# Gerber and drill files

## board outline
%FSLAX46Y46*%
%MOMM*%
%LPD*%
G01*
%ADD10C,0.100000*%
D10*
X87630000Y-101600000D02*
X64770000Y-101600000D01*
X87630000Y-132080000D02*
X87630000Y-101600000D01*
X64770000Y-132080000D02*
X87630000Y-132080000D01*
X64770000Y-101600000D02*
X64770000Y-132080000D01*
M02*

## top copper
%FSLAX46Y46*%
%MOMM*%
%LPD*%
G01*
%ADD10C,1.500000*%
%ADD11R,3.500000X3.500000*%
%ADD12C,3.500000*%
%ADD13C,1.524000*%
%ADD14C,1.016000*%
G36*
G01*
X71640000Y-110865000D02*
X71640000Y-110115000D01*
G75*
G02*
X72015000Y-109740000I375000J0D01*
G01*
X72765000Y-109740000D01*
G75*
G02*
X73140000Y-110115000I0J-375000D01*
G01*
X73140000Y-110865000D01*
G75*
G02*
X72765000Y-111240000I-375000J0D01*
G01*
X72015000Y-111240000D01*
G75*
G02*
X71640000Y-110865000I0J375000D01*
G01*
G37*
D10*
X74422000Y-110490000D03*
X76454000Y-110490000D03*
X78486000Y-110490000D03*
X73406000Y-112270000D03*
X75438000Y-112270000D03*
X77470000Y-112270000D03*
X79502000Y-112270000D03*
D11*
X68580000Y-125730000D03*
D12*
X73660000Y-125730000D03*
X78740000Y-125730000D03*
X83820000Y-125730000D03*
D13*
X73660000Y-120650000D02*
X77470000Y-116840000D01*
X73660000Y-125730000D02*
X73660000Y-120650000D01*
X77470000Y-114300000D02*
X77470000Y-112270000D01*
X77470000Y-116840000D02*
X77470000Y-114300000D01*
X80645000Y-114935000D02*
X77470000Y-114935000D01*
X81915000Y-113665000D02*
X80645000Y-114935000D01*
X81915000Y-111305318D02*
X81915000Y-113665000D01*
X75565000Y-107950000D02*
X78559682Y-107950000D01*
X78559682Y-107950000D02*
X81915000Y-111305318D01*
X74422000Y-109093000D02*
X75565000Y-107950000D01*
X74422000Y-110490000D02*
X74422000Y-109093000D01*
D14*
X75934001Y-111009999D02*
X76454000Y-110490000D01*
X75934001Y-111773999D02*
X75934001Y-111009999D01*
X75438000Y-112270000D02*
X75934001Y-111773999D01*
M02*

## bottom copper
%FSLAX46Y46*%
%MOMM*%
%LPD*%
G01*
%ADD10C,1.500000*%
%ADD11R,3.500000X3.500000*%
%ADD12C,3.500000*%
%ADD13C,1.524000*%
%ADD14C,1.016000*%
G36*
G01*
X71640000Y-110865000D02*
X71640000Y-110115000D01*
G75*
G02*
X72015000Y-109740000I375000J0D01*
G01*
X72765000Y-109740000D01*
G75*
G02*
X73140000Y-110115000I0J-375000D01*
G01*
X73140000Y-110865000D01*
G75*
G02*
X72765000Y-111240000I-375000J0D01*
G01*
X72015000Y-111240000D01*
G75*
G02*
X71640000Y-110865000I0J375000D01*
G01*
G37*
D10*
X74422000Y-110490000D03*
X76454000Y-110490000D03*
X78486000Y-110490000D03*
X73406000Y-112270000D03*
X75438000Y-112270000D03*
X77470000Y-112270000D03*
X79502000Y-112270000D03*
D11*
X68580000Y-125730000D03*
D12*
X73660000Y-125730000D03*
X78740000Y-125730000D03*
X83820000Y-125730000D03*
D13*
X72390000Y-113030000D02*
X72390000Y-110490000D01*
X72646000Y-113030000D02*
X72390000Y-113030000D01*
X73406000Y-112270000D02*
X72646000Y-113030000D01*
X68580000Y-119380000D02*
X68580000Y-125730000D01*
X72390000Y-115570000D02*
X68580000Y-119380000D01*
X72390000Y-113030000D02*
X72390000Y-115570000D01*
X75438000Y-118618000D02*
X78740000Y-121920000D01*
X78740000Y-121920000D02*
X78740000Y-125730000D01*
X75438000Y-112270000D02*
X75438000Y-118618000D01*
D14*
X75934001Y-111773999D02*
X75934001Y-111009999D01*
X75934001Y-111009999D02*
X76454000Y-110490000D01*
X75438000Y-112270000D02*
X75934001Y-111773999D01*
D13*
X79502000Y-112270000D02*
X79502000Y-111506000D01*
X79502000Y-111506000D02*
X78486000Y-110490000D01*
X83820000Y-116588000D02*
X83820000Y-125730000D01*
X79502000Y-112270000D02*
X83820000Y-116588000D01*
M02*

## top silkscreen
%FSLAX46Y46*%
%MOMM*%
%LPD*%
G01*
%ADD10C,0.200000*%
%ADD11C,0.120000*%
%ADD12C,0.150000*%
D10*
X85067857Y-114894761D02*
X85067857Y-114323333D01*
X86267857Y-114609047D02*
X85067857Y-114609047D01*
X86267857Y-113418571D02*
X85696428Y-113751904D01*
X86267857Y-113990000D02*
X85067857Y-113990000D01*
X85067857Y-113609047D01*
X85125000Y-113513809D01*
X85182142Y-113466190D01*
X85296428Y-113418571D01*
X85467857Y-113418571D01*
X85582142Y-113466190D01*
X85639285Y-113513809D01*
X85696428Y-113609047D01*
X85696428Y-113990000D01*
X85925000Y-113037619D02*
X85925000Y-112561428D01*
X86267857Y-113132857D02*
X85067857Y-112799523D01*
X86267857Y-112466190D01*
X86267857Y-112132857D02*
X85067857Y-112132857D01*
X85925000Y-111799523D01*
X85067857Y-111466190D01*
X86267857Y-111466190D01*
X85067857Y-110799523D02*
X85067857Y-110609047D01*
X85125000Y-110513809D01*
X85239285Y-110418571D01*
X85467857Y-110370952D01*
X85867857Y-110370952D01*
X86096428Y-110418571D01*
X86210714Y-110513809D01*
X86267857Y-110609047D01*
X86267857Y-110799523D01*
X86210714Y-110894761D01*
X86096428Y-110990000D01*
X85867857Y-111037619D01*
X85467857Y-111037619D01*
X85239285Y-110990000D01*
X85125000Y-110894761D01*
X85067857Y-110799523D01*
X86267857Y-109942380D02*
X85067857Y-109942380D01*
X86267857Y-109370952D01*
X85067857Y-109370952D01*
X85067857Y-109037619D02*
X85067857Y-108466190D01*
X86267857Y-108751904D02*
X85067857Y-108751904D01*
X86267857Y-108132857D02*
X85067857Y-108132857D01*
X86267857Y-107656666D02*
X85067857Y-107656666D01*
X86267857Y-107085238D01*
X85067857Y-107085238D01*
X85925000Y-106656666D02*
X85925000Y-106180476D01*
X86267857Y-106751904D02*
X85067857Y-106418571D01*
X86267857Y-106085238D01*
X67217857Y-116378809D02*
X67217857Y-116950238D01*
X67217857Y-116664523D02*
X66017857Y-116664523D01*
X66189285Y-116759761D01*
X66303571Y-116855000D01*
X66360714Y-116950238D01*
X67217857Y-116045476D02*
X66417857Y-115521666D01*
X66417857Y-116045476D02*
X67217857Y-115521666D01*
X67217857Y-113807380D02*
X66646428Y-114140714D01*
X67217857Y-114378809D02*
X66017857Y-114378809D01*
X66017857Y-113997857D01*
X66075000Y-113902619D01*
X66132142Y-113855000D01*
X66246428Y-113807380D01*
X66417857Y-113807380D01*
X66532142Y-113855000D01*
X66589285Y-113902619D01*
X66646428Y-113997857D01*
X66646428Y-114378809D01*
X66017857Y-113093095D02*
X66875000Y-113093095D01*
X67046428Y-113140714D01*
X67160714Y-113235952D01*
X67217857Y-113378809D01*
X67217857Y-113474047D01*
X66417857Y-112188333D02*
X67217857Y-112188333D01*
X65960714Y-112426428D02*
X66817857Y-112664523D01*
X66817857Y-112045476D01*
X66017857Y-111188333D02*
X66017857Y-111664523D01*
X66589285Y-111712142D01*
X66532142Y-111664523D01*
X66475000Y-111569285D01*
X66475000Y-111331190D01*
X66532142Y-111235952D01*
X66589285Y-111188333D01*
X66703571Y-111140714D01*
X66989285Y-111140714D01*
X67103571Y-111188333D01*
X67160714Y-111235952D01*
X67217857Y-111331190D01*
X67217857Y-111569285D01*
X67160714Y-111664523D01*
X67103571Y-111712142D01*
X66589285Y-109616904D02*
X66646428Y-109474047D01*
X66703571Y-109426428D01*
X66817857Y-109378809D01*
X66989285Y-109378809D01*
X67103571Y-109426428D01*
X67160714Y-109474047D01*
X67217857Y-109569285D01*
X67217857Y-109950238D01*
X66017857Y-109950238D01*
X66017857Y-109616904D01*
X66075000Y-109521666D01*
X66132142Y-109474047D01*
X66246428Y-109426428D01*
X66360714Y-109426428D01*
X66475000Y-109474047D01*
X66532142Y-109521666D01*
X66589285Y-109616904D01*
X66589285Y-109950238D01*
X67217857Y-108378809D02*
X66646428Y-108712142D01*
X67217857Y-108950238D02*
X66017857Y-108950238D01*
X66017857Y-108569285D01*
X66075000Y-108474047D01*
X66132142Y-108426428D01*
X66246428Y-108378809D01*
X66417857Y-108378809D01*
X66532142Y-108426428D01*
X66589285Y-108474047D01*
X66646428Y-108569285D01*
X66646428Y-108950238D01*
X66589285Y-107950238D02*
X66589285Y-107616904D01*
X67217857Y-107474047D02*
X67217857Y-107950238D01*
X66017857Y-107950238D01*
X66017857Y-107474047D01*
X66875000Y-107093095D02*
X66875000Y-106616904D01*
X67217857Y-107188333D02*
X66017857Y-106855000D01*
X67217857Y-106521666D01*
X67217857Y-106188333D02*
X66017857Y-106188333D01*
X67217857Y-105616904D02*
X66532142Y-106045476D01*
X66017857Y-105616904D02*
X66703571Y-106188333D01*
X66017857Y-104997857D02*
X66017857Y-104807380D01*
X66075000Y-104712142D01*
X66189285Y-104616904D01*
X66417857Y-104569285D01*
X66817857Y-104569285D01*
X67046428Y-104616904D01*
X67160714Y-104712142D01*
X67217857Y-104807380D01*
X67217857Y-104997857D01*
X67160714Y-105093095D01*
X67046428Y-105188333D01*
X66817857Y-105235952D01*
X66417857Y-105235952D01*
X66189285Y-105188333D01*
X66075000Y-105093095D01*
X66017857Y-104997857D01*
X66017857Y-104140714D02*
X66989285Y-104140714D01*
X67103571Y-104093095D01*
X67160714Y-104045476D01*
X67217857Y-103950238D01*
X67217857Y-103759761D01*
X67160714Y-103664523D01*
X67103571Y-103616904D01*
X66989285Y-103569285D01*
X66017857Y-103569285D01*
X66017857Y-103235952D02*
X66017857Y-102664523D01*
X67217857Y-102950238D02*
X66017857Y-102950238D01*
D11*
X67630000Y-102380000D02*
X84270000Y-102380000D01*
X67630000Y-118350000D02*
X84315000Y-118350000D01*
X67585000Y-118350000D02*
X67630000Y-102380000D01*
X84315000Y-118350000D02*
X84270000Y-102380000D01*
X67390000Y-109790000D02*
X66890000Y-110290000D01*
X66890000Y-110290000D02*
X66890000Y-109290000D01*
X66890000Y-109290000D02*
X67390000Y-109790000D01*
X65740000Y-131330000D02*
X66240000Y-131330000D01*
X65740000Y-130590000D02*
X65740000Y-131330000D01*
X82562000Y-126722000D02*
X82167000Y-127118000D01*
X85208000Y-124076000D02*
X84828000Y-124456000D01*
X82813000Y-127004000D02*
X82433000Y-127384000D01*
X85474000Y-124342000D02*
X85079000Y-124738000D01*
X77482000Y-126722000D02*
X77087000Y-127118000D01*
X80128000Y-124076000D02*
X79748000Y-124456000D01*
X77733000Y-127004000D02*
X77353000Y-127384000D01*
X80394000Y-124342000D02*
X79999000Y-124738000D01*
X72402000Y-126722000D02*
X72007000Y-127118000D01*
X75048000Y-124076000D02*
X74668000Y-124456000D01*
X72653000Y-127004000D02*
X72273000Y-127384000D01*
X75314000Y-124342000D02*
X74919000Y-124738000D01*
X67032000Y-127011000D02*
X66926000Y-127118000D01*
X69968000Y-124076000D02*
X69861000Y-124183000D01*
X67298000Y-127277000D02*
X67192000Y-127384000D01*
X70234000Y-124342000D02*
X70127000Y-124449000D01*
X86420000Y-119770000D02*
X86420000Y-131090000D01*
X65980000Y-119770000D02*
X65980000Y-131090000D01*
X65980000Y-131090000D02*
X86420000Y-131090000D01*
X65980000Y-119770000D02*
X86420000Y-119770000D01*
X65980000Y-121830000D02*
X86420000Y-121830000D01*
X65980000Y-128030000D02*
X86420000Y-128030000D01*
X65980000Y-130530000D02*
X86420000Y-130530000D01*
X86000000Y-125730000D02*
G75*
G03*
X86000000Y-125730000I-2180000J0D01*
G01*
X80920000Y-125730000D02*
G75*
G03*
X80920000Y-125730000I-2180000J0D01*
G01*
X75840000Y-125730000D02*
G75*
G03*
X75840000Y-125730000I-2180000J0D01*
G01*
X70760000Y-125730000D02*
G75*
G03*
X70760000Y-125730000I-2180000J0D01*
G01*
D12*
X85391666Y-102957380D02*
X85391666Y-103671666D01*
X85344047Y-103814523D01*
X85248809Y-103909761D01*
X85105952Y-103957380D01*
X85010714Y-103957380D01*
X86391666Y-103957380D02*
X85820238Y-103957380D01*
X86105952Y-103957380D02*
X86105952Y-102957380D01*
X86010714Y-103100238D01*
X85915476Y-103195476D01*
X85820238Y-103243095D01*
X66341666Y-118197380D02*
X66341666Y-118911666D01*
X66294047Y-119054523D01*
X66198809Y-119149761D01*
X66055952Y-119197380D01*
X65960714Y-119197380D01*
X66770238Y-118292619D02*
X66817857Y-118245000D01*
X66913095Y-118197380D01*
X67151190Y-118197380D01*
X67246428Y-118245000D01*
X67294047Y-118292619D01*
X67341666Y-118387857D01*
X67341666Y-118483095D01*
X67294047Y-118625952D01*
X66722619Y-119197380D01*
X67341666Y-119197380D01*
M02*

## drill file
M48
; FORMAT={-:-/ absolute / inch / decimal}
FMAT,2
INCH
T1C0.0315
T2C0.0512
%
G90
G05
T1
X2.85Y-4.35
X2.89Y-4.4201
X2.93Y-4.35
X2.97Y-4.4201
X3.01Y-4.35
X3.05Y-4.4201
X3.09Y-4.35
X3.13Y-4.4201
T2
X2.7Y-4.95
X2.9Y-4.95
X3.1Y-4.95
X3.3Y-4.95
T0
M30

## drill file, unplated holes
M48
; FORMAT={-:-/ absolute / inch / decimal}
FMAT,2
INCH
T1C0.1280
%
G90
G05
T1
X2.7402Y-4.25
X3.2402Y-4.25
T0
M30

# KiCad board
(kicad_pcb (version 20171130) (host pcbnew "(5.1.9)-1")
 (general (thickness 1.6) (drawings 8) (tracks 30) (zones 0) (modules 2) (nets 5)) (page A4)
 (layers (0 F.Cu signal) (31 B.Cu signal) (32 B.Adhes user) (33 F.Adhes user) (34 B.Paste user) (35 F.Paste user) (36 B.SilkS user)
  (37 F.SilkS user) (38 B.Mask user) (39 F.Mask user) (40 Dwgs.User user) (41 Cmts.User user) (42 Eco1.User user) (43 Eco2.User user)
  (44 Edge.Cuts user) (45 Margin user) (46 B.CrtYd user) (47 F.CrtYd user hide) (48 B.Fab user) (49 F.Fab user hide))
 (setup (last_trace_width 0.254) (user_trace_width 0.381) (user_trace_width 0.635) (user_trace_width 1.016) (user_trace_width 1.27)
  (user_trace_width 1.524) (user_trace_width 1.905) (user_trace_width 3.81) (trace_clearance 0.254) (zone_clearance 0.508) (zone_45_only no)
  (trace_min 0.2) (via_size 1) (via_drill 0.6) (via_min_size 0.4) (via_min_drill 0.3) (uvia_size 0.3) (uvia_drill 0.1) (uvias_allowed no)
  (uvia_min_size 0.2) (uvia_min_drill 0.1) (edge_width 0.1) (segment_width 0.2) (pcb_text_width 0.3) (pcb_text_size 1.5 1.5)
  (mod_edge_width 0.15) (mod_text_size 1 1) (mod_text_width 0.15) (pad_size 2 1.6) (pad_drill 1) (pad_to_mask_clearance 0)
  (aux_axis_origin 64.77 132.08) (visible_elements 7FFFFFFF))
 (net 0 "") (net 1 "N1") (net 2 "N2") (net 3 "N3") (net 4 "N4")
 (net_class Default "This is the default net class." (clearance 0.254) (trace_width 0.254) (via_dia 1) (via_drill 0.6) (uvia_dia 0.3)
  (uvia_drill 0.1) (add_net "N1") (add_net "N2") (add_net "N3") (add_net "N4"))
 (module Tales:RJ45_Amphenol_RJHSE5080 (layer F.Cu) (at 72.39 110.49)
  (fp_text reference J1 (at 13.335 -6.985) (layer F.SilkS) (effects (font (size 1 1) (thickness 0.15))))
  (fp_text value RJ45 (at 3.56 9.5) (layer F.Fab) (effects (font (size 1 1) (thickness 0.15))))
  (fp_line (start -4.76 -8.11) (end 11.88 -8.11) (layer F.SilkS) (width 0.12))
  (fp_line (start -4.76 7.86) (end 11.925 7.86) (layer F.SilkS) (width 0.12))
  (fp_line (start -4.805 7.86) (end -4.76 -8.11) (layer F.SilkS) (width 0.12))
  (fp_line (start 11.925 7.86) (end 11.88 -8.11) (layer F.SilkS) (width 0.12))
  (fp_line (start -5 -0.7) (end -5.5 -0.2) (layer F.SilkS) (width 0.12))
  (fp_line (start -5.5 -0.2) (end -5.5 -1.2) (layer F.SilkS) (width 0.12))
  (fp_line (start -5.5 -1.2) (end -5 -0.7) (layer F.SilkS) (width 0.12))
  (pad 1 thru_hole roundrect (at 0 0) (size 1.5 1.5) (drill 0.8) (layers *.Cu *.Mask) (roundrect_rratio 0.25) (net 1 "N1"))
  (pad 3 thru_hole circle (at 2.032 0) (size 1.5 1.5) (drill 0.8) (layers *.Cu *.Mask) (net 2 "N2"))
  (pad 5 thru_hole circle (at 4.064 0) (size 1.5 1.5) (drill 0.8) (layers *.Cu *.Mask) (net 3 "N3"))
  (pad 7 thru_hole circle (at 6.096 0) (size 1.5 1.5) (drill 0.8) (layers *.Cu *.Mask) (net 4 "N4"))
  (pad 2 thru_hole circle (at 1.016 1.78) (size 1.5 1.5) (drill 0.8) (layers *.Cu *.Mask) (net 1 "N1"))
  (pad 4 thru_hole circle (at 3.048 1.78) (size 1.5 1.5) (drill 0.8) (layers *.Cu *.Mask) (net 3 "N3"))
  (pad 6 thru_hole circle (at 5.08 1.78) (size 1.5 1.5) (drill 0.8) (layers *.Cu *.Mask) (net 2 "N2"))
  (pad 8 thru_hole circle (at 7.112 1.78) (size 1.5 1.5) (drill 0.8) (layers *.Cu *.Mask) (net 4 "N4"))
  (pad "" np_thru_hole circle (at -2.79 -2.54) (size 3.25 3.25) (drill 3.25) (layers *.Cu *.Mask))
  (pad "" np_thru_hole circle (at 9.91 -2.54) (size 3.25 3.25) (drill 3.25) (layers *.Cu *.Mask)))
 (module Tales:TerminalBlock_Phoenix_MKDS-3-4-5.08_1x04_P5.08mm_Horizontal (layer F.Cu) (at 68.58 125.73)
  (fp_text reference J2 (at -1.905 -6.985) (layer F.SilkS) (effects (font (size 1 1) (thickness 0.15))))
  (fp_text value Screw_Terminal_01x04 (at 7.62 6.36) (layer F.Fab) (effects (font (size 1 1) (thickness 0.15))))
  (fp_line (start -2.84 5.6) (end -2.34 5.6) (layer F.SilkS) (width 0.12))
  (fp_line (start -2.84 4.86) (end -2.84 5.6) (layer F.SilkS) (width 0.12))
  (fp_line (start 13.982 0.992) (end 13.587 1.388) (layer F.SilkS) (width 0.12))
  (fp_line (start 16.628 -1.654) (end 16.248 -1.274) (layer F.SilkS) (width 0.12))
  (fp_line (start 14.233 1.274) (end 13.853 1.654) (layer F.SilkS) (width 0.12))
  (fp_line (start 16.894 -1.388) (end 16.499 -0.992) (layer F.SilkS) (width 0.12))
  (fp_line (start 8.902 0.992) (end 8.507 1.388) (layer F.SilkS) (width 0.12))
  (fp_line (start 11.548 -1.654) (end 11.168 -1.274) (layer F.SilkS) (width 0.12))
  (fp_line (start 9.153 1.274) (end 8.773 1.654) (layer F.SilkS) (width 0.12))
  (fp_line (start 11.814 -1.388) (end 11.419 -0.992) (layer F.SilkS) (width 0.12))
  (fp_line (start 3.822 0.992) (end 3.427 1.388) (layer F.SilkS) (width 0.12))
  (fp_line (start 6.468 -1.654) (end 6.088 -1.274) (layer F.SilkS) (width 0.12))
  (fp_line (start 4.073 1.274) (end 3.693 1.654) (layer F.SilkS) (width 0.12))
  (fp_line (start 6.734 -1.388) (end 6.339 -0.992) (layer F.SilkS) (width 0.12))
  (fp_line (start -1.548 1.281) (end -1.654 1.388) (layer F.SilkS) (width 0.12))
  (fp_line (start 1.388 -1.654) (end 1.281 -1.547) (layer F.SilkS) (width 0.12))
  (fp_line (start -1.282 1.547) (end -1.388 1.654) (layer F.SilkS) (width 0.12))
  (fp_line (start 1.654 -1.388) (end 1.547 -1.281) (layer F.SilkS) (width 0.12))
  (fp_line (start 17.84 -5.96) (end 17.84 5.36) (layer F.SilkS) (width 0.12))
  (fp_line (start -2.6 -5.96) (end -2.6 5.36) (layer F.SilkS) (width 0.12))
  (fp_line (start -2.6 5.36) (end 17.84 5.36) (layer F.SilkS) (width 0.12))
  (fp_line (start -2.6 -5.96) (end 17.84 -5.96) (layer F.SilkS) (width 0.12))
  (fp_line (start -2.6 -3.9) (end 17.84 -3.9) (layer F.SilkS) (width 0.12))
  (fp_line (start -2.6 2.3) (end 17.84 2.3) (layer F.SilkS) (width 0.12))
  (fp_line (start -2.6 4.8) (end 17.84 4.8) (layer F.SilkS) (width 0.12))
  (fp_circle (center 15.24 0) (end 17.42 0) (layer F.SilkS) (width 0.12))
  (fp_circle (center 10.16 0) (end 12.34 0) (layer F.SilkS) (width 0.12))
  (fp_circle (center 5.08 0) (end 7.26 0) (layer F.SilkS) (width 0.12))
  (fp_circle (center 0 0) (end 2.18 0) (layer F.SilkS) (width 0.12))
  (pad 1 thru_hole rect (at 0 0) (size 3.5 3.5) (drill 1.3) (layers *.Cu *.Mask) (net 1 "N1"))
  (pad 2 thru_hole circle (at 5.08 0) (size 3.5 3.5) (drill 1.3) (layers *.Cu *.Mask) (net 2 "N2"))
  (pad 3 thru_hole circle (at 10.16 0) (size 3.5 3.5) (drill 1.3) (layers *.Cu *.Mask) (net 3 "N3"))
  (pad 4 thru_hole circle (at 15.24 0) (size 3.5 3.5) (drill 1.3) (layers *.Cu *.Mask) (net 4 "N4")))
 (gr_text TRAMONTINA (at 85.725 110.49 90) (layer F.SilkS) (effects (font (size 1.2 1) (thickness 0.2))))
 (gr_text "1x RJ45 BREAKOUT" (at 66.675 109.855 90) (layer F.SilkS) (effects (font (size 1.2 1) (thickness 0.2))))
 (gr_line (start 87.63 101.6) (end 64.77 101.6) (layer Edge.Cuts) (width 0.1))
 (gr_line (start 87.63 132.08) (end 87.63 101.6) (layer Edge.Cuts) (width 0.1))
 (gr_line (start 64.77 132.08) (end 87.63 132.08) (layer Edge.Cuts) (width 0.1))
 (gr_line (start 64.77 101.6) (end 64.77 132.08) (layer Edge.Cuts) (width 0.1))
 (segment (start 72.39 113.03) (end 72.39 110.49) (width 1.524) (layer B.Cu) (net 1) (status 20))
 (segment (start 72.646 113.03) (end 72.39 113.03) (width 1.524) (layer B.Cu) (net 1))
 (segment (start 73.406 112.27) (end 72.646 113.03) (width 1.524) (layer B.Cu) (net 1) (status 10))
 (segment (start 68.58 119.38) (end 68.58 125.73) (width 1.524) (layer B.Cu) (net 1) (status 20))
 (segment (start 72.39 115.57) (end 68.58 119.38) (width 1.524) (layer B.Cu) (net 1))
 (segment (start 72.39 113.03) (end 72.39 115.57) (width 1.524) (layer B.Cu) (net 1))
 (segment (start 73.66 120.65) (end 77.47 116.84) (width 1.524) (layer F.Cu) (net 2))
 (segment (start 73.66 125.73) (end 73.66 120.65) (width 1.524) (layer F.Cu) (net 2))
 (segment (start 77.47 114.3) (end 77.47 112.27) (width 1.524) (layer F.Cu) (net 2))
 (segment (start 77.47 116.84) (end 77.47 114.3) (width 1.524) (layer F.Cu) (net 2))
 (segment (start 80.645 114.935) (end 77.47 114.935) (width 1.524) (layer F.Cu) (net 2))
 (segment (start 81.915 113.665) (end 80.645 114.935) (width 1.524) (layer F.Cu) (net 2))
 (segment (start 81.915 111.305318) (end 81.915 113.665) (width 1.524) (layer F.Cu) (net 2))
 (segment (start 75.565 107.95) (end 78.559682 107.95) (width 1.524) (layer F.Cu) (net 2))
 (segment (start 78.559682 107.95) (end 81.915 111.305318) (width 1.524) (layer F.Cu) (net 2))
 (segment (start 74.422 109.093) (end 75.565 107.95) (width 1.524) (layer F.Cu) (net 2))
 (segment (start 74.422 110.49) (end 74.422 109.093) (width 1.524) (layer F.Cu) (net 2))
 (segment (start 75.438 118.618) (end 78.74 121.92) (width 1.524) (layer B.Cu) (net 3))
 (segment (start 78.74 121.92) (end 78.74 125.73) (width 1.524) (layer B.Cu) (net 3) (status 20))
 (segment (start 75.438 112.27) (end 75.438 118.618) (width 1.524) (layer B.Cu) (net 3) (status 10))
 (segment (start 75.934001 111.773999) (end 75.934001 111.009999) (width 1.016) (layer B.Cu) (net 3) (status 30))
 (segment (start 75.934001 111.009999) (end 76.454 110.49) (width 1.016) (layer B.Cu) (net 3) (status 30))
 (segment (start 75.438 112.27) (end 75.934001 111.773999) (width 1.016) (layer B.Cu) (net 3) (status 30))
 (segment (start 75.934001 111.009999) (end 76.454 110.49) (width 1.016) (layer F.Cu) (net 3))
 (segment (start 75.934001 111.773999) (end 75.934001 111.009999) (width 1.016) (layer F.Cu) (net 3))
 (segment (start 75.438 112.27) (end 75.934001 111.773999) (width 1.016) (layer F.Cu) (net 3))
 (segment (start 79.502 112.27) (end 79.502 111.506) (width 1.524) (layer B.Cu) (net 4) (status 10))
 (segment (start 79.502 111.506) (end 78.486 110.49) (width 1.524) (layer B.Cu) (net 4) (status 20))
 (segment (start 83.82 116.588) (end 83.82 125.73) (width 1.524) (layer B.Cu) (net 4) (status 20))
 (segment (start 79.502 112.27) (end 83.82 116.588) (width 1.524) (layer B.Cu) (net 4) (status 10)))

